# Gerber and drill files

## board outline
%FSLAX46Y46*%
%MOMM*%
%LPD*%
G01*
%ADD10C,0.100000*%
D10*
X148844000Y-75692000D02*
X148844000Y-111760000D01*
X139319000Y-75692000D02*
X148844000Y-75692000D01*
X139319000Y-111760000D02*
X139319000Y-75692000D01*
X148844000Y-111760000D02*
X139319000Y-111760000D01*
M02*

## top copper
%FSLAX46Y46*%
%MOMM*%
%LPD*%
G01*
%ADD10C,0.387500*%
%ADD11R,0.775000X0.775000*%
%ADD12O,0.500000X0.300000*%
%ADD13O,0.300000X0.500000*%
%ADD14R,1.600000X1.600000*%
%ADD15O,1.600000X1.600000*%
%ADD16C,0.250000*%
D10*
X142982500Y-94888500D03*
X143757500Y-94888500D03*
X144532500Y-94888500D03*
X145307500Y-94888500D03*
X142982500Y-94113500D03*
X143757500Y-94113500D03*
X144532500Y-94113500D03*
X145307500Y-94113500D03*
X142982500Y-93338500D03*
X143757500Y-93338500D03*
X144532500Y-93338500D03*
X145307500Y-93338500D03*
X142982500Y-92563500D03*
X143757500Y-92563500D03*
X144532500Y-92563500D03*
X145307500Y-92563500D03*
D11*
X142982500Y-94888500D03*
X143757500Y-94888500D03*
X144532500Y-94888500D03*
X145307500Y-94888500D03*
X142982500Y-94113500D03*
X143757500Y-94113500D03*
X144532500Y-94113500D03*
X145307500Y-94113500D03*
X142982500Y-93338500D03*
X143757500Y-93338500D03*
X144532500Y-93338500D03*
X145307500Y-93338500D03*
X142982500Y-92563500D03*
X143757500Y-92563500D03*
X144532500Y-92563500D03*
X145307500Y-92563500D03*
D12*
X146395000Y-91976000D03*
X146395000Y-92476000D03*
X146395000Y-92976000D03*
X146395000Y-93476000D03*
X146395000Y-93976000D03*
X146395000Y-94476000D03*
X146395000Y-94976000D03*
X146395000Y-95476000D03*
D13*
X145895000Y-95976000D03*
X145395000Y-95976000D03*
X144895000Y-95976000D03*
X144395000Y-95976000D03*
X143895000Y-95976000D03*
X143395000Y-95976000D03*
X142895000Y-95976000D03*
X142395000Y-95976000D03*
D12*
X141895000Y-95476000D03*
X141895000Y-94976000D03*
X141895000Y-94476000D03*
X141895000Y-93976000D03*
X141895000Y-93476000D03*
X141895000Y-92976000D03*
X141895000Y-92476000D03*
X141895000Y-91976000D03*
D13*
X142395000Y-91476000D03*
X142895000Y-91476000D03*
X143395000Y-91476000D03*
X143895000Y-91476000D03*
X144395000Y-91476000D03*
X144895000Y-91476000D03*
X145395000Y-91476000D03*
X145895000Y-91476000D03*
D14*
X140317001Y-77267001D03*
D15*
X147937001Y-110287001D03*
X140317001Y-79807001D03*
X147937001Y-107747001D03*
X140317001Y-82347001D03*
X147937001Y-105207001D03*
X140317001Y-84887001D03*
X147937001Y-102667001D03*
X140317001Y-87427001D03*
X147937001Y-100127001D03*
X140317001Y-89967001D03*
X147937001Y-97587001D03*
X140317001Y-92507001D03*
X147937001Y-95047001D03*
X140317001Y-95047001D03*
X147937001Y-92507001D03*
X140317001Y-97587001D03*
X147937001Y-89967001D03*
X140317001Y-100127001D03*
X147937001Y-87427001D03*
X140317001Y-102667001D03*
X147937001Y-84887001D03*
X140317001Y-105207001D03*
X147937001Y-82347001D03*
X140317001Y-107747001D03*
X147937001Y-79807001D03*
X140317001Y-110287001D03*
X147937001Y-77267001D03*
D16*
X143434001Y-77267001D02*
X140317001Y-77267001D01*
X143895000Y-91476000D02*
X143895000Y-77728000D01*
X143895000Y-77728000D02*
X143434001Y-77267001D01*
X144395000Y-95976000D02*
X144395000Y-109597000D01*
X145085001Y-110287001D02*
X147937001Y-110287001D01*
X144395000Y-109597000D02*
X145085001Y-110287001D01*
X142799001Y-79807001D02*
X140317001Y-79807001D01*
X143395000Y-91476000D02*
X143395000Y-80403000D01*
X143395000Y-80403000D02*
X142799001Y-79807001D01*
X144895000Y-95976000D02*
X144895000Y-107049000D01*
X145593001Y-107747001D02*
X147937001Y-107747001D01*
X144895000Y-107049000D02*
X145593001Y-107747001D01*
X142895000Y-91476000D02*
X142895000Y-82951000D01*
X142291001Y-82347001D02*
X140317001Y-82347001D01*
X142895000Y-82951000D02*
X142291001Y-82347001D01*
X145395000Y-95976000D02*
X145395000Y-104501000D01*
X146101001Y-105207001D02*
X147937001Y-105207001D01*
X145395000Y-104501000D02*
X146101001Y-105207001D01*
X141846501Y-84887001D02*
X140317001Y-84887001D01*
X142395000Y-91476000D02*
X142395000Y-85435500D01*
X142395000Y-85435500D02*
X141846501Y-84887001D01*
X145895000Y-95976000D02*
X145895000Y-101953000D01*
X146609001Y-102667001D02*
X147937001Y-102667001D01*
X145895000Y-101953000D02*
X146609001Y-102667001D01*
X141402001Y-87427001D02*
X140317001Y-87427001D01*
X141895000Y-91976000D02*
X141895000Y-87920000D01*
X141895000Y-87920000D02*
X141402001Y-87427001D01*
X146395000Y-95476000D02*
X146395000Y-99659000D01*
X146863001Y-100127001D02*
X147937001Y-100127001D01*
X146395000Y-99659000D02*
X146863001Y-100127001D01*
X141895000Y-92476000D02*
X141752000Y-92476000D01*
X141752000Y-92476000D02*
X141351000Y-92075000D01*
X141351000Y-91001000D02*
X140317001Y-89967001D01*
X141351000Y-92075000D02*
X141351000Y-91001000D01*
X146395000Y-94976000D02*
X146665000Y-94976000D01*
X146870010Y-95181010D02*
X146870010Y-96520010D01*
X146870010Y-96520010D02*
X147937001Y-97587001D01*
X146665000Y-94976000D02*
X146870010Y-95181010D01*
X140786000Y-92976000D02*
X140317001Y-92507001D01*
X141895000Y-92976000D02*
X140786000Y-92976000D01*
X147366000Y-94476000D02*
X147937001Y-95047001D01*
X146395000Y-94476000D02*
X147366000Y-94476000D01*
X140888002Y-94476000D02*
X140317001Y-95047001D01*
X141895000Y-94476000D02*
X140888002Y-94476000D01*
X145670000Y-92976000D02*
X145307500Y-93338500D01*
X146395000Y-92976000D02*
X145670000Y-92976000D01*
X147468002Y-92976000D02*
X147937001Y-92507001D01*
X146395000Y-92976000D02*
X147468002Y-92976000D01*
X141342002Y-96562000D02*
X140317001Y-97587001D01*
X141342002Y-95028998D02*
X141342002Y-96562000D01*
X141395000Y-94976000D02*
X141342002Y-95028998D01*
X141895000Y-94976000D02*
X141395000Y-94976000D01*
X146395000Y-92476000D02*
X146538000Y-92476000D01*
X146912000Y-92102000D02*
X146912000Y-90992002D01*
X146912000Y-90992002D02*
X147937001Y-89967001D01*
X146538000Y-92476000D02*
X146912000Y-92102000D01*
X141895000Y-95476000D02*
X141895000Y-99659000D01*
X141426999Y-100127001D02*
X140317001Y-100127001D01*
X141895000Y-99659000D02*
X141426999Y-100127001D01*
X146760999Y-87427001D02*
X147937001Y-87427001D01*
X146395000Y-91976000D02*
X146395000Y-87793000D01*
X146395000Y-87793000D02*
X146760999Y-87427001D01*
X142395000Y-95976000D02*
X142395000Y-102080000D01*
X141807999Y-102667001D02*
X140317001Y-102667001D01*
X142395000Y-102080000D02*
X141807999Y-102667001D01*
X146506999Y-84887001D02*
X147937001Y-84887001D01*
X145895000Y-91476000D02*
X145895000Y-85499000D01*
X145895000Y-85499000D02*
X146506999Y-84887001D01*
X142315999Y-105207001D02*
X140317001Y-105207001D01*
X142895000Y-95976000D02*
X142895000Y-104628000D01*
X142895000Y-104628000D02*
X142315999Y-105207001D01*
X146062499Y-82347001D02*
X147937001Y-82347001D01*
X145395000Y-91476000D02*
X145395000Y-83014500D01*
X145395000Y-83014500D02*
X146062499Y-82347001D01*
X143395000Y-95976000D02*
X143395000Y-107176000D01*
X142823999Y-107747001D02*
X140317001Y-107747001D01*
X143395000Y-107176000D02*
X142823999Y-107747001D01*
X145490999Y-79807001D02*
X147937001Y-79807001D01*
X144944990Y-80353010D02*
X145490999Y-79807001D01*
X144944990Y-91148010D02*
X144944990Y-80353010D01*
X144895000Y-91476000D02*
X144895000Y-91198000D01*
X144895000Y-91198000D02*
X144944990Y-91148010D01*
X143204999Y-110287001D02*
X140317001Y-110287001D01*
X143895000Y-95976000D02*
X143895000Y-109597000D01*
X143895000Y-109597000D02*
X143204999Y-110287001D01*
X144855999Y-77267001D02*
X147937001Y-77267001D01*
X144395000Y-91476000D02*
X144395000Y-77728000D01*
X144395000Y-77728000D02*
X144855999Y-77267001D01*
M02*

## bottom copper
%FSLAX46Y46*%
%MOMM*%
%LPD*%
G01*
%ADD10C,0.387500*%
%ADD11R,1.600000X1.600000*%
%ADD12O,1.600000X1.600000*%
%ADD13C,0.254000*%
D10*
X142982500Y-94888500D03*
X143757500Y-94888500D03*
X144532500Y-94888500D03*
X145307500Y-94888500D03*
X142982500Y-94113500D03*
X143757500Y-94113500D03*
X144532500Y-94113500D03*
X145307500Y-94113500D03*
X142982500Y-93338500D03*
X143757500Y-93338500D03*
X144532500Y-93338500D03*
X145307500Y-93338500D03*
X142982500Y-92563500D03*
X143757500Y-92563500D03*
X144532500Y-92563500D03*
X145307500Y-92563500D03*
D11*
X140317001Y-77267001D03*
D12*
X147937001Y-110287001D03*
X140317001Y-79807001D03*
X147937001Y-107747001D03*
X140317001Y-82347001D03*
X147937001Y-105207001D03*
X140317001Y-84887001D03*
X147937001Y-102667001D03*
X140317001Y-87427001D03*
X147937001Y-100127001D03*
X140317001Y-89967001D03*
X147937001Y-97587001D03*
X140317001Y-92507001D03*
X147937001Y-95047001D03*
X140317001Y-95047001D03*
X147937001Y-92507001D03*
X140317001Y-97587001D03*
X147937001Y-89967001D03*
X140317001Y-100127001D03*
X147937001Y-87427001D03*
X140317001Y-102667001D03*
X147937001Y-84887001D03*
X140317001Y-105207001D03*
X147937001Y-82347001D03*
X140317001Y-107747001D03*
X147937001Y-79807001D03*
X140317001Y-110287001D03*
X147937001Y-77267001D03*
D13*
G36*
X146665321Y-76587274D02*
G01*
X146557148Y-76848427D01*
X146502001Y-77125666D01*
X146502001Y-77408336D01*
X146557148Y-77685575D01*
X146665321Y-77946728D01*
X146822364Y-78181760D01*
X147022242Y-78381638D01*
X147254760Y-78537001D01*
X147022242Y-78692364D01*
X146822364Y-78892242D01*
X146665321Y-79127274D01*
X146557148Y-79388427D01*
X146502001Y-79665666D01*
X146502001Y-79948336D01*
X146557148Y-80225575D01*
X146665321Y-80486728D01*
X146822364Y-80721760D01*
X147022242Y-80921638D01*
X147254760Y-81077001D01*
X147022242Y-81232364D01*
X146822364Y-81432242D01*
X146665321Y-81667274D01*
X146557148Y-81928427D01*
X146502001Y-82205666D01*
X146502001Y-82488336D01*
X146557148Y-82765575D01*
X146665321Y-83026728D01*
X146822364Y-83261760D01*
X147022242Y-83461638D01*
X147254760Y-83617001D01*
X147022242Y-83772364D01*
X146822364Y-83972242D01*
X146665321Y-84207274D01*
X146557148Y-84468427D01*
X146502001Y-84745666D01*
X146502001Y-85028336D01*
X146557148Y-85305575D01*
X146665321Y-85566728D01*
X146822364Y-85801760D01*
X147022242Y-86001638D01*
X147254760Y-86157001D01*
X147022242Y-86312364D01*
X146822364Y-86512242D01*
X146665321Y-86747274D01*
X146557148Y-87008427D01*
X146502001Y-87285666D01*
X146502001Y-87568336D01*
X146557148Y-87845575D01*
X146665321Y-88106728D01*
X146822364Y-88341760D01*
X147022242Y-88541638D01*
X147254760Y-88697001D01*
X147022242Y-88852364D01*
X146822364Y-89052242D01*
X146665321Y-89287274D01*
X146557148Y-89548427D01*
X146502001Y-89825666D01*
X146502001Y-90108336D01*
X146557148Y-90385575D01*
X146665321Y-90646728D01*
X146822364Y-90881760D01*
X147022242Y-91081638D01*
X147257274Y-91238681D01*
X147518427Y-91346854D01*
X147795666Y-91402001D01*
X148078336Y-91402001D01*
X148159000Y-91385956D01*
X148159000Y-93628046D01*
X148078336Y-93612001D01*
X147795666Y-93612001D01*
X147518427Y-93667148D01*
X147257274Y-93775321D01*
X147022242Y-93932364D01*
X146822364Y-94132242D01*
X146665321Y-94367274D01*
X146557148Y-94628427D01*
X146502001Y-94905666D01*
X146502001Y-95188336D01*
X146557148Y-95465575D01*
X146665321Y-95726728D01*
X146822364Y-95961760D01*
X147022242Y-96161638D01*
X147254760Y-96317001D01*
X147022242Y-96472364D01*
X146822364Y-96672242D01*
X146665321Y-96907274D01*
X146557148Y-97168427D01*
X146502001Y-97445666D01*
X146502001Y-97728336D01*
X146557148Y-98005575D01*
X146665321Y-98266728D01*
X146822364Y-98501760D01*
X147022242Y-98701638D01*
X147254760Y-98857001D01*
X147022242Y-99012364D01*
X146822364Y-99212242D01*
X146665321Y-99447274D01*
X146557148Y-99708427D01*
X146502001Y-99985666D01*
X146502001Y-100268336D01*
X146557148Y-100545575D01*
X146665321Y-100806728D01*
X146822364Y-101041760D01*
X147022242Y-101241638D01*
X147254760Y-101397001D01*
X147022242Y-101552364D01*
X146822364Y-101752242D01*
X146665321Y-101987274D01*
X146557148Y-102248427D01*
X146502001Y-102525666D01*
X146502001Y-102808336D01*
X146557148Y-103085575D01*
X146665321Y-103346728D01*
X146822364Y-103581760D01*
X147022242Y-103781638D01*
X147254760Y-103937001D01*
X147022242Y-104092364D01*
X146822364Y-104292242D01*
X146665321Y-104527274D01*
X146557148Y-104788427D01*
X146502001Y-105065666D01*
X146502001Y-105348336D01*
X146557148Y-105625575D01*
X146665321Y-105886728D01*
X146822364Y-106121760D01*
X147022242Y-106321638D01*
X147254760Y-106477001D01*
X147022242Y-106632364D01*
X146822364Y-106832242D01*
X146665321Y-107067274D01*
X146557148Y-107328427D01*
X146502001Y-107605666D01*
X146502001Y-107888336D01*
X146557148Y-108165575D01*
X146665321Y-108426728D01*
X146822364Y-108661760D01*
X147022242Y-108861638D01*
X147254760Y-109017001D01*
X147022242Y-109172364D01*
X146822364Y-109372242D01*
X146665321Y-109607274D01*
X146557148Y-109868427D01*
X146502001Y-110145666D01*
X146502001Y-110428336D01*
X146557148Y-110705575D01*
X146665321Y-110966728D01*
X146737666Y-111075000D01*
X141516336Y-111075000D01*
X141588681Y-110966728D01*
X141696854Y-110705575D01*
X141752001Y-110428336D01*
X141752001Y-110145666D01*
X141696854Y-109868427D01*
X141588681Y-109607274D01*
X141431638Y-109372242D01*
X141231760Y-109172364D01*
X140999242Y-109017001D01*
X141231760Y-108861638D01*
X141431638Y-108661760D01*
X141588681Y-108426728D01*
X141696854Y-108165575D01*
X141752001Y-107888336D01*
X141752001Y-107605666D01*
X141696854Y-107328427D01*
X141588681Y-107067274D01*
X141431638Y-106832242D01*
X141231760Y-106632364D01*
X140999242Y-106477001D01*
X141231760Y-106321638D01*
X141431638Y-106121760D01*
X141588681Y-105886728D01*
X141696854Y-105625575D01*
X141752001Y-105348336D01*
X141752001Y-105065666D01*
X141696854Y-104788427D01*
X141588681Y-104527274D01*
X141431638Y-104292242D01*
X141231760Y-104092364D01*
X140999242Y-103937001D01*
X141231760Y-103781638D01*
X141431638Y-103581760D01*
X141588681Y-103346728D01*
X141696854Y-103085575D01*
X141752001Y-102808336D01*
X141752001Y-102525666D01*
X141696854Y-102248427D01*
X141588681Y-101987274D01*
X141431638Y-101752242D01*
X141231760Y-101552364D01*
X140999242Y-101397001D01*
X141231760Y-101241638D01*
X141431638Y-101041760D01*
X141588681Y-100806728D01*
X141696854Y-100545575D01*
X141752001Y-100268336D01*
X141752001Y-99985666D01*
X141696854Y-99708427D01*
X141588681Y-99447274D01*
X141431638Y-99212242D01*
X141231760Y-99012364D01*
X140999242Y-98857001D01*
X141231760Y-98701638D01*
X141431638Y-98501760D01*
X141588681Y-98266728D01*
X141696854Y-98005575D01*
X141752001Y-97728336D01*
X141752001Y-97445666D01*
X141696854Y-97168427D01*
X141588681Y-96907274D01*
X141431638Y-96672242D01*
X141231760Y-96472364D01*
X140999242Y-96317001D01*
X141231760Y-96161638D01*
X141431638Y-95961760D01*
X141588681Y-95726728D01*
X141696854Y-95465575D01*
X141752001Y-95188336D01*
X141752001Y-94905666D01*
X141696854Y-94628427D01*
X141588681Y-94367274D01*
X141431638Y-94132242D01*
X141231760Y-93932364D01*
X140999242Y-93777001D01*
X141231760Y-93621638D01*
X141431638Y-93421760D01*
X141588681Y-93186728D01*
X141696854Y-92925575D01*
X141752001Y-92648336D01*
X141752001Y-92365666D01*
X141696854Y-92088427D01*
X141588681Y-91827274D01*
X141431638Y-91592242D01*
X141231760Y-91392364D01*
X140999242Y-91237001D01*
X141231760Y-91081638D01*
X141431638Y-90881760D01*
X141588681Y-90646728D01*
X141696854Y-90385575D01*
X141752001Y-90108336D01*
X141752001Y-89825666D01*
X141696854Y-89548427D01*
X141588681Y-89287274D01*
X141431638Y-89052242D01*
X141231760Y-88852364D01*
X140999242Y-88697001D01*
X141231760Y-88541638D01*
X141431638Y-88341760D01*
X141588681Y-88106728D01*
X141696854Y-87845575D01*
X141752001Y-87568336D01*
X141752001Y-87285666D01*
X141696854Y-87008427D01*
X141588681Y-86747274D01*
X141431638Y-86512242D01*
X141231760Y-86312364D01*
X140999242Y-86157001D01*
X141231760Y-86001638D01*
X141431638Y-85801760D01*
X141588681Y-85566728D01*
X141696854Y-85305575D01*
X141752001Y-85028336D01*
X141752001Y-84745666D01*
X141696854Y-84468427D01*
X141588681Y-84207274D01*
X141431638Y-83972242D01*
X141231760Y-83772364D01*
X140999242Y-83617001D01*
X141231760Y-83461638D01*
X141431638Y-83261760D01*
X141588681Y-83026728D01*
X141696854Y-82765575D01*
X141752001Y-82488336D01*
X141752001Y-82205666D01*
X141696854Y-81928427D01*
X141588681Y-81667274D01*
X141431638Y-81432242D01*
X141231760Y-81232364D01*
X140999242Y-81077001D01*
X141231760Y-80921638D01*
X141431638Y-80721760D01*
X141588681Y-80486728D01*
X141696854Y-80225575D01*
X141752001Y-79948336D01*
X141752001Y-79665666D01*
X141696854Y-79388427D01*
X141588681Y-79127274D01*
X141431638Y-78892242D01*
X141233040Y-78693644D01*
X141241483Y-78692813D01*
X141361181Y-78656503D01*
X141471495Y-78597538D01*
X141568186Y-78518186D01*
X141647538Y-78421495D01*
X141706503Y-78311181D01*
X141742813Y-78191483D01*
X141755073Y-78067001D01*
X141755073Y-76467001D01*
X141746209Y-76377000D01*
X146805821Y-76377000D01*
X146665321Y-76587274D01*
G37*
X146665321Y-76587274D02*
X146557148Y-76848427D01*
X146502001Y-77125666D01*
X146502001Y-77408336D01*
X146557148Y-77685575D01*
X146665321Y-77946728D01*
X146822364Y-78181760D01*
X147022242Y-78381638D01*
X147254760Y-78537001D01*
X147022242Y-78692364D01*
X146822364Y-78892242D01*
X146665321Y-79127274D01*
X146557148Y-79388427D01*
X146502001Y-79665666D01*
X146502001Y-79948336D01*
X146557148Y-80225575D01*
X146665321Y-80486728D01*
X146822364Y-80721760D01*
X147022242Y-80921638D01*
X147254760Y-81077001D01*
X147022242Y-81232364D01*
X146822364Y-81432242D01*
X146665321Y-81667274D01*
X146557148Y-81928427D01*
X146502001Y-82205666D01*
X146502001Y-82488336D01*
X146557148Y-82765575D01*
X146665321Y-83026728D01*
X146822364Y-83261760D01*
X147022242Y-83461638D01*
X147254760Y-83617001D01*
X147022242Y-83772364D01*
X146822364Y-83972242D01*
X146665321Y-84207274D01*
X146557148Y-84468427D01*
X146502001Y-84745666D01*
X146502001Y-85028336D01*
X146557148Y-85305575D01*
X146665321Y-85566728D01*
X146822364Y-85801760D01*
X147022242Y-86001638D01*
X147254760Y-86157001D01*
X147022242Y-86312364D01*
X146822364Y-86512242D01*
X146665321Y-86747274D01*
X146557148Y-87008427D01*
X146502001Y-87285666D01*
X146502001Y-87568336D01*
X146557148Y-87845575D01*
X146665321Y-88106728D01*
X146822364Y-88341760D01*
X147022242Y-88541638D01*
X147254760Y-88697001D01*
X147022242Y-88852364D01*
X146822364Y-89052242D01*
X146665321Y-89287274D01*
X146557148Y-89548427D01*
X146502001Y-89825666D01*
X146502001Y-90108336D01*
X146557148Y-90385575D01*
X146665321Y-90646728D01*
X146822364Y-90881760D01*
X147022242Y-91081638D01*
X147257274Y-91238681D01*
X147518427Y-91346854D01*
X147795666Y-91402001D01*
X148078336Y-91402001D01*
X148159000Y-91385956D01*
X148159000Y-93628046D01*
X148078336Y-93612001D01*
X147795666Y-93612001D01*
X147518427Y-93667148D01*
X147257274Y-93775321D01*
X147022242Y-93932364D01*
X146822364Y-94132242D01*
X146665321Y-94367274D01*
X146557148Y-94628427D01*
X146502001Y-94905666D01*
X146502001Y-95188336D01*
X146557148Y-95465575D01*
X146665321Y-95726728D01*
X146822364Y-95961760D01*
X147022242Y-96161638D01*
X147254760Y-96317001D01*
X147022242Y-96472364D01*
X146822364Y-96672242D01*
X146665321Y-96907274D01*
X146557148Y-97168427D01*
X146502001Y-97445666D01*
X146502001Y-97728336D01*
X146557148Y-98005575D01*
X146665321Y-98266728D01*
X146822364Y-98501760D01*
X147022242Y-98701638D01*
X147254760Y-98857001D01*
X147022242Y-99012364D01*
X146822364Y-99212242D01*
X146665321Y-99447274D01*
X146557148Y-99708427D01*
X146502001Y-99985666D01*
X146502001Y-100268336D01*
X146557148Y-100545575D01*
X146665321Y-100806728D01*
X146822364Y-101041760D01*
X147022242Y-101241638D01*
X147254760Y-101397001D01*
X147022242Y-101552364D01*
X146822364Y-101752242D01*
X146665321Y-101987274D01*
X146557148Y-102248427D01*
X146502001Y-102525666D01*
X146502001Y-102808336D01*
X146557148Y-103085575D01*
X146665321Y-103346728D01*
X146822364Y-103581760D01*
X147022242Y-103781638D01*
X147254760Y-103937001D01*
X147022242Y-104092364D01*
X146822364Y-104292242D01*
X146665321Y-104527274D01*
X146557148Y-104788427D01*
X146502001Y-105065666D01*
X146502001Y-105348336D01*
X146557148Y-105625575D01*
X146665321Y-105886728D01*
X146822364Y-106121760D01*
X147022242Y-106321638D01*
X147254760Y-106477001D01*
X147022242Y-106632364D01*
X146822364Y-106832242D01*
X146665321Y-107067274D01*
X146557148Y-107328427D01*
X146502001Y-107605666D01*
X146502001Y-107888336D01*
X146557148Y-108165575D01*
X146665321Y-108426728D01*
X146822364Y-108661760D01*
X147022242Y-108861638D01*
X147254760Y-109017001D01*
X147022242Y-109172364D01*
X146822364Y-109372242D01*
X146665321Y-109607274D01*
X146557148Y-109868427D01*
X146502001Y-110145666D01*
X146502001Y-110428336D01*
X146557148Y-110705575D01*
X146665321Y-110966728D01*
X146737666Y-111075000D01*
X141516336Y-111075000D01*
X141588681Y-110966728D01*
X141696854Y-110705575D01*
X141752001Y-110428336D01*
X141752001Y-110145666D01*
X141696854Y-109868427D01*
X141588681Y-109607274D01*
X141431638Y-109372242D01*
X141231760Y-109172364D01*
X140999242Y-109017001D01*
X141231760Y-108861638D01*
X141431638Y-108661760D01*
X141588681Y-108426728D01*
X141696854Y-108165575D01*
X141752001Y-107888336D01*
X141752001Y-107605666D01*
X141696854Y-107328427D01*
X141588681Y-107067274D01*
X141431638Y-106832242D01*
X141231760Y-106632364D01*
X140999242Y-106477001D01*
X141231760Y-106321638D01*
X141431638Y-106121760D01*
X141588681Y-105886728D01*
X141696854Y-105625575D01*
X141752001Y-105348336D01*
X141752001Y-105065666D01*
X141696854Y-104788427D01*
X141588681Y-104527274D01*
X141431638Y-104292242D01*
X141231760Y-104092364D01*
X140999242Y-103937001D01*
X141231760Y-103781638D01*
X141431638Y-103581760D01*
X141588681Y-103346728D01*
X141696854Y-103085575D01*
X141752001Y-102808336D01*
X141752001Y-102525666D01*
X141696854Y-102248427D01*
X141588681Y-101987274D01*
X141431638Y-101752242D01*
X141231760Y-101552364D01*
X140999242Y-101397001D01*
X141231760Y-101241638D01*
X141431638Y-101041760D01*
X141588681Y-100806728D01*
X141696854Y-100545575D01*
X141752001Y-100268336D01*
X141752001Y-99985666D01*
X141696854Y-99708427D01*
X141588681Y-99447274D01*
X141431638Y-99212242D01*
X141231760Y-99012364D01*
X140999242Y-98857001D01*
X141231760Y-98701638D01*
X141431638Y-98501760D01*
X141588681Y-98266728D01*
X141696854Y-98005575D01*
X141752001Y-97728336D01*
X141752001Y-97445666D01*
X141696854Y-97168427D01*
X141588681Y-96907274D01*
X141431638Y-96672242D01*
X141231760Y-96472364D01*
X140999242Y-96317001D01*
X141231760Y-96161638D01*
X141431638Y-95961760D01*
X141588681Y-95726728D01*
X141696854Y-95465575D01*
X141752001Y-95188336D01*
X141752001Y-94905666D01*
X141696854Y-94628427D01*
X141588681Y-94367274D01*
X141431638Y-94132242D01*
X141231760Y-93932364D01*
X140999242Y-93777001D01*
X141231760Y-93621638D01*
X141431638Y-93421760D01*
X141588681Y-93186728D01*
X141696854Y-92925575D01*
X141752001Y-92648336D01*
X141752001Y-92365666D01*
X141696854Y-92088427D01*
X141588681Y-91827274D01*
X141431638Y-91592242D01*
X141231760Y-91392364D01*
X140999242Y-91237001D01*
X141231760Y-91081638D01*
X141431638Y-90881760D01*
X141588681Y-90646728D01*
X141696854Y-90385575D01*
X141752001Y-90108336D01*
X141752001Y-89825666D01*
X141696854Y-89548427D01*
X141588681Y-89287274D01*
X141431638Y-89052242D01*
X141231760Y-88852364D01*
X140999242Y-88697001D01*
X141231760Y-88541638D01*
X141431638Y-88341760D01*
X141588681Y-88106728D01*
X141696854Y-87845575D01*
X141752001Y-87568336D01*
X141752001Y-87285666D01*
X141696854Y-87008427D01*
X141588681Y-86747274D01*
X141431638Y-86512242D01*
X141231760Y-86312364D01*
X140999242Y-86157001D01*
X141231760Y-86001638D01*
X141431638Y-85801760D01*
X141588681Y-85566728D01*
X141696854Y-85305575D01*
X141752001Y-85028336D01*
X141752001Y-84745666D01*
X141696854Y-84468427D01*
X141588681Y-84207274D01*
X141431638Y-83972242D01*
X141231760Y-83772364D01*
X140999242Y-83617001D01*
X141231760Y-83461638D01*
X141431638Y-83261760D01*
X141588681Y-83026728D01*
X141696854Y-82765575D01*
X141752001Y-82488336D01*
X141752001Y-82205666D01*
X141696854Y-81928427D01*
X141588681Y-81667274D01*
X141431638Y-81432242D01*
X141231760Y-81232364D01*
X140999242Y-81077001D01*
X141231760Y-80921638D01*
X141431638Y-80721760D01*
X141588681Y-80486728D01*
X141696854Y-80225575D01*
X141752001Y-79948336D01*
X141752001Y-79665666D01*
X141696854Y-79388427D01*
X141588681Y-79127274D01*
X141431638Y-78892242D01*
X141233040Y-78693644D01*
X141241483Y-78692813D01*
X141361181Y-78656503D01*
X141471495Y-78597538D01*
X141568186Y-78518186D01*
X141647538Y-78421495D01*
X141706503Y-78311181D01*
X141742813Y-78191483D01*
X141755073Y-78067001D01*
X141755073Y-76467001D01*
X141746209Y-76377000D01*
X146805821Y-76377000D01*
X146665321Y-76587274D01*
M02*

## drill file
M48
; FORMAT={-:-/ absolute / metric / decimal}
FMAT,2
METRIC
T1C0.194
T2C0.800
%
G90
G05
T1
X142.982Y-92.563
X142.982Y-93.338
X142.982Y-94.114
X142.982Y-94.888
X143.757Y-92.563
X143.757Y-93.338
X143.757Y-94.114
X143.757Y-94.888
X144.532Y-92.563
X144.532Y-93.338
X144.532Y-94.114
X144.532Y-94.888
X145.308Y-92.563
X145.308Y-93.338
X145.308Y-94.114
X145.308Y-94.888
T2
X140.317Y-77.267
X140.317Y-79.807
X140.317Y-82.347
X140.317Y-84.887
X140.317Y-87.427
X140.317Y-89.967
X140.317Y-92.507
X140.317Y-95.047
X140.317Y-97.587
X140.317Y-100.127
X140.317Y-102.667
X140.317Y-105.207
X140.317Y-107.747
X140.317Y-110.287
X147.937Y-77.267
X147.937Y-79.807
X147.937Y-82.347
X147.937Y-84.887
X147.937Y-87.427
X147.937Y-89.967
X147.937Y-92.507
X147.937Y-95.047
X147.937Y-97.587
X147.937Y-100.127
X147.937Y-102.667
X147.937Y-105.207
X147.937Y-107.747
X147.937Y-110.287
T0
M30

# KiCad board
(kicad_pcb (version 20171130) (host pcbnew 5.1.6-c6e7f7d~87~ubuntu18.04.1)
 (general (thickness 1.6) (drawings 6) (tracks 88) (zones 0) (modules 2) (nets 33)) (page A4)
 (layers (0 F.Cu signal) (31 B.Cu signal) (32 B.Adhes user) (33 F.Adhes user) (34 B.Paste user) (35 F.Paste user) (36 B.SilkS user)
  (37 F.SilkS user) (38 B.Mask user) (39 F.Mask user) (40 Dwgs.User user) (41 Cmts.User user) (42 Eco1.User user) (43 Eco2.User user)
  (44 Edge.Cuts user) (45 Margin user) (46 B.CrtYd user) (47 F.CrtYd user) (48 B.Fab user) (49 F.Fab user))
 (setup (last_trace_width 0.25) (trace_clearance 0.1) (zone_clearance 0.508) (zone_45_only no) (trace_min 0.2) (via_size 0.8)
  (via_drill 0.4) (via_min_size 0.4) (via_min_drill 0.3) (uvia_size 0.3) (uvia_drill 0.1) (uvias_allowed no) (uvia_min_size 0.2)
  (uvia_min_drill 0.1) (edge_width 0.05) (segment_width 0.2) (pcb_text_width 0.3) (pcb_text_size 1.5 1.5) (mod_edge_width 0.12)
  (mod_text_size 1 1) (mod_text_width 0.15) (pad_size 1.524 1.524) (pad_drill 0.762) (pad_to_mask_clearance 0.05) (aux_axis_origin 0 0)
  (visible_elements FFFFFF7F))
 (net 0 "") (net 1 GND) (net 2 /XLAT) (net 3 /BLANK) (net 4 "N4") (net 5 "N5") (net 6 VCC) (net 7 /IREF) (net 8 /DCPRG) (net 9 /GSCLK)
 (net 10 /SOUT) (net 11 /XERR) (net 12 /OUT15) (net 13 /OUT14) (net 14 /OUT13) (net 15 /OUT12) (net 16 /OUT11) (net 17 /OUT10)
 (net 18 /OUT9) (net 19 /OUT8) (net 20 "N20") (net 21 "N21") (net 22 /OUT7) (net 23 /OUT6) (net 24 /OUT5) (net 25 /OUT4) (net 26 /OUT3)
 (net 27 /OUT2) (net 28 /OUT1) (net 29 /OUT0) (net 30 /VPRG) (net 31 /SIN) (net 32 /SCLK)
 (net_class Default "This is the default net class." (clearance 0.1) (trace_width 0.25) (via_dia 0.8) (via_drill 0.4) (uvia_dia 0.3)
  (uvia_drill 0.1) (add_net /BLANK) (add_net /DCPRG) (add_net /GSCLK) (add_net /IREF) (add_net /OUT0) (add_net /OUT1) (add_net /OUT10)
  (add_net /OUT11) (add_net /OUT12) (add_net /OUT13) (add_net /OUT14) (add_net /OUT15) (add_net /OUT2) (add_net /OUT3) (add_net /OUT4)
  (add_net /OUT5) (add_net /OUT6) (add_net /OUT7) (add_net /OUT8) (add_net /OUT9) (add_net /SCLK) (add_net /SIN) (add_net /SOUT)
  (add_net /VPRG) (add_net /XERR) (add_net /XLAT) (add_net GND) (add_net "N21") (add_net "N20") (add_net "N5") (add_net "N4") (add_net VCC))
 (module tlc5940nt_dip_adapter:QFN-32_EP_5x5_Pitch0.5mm (layer F.Cu) (at 144.145 93.726 270)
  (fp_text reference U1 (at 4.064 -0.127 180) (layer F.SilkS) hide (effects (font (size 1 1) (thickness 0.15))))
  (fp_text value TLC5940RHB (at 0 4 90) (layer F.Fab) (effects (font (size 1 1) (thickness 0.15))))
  (pad 33 thru_hole circle (at 1.1625 1.1625 270) (size 0.3875 0.3875) (drill 0.19375) (layers *.Cu *.Mask) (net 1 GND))
  (pad 33 thru_hole circle (at 1.1625 0.3875 270) (size 0.3875 0.3875) (drill 0.19375) (layers *.Cu *.Mask) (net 1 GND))
  (pad 33 thru_hole circle (at 1.1625 -0.3875 270) (size 0.3875 0.3875) (drill 0.19375) (layers *.Cu *.Mask) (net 1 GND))
  (pad 33 thru_hole circle (at 1.1625 -1.1625 270) (size 0.3875 0.3875) (drill 0.19375) (layers *.Cu *.Mask) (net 1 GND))
  (pad 33 thru_hole circle (at 0.3875 1.1625 270) (size 0.3875 0.3875) (drill 0.19375) (layers *.Cu *.Mask) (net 1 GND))
  (pad 33 thru_hole circle (at 0.3875 0.3875 270) (size 0.3875 0.3875) (drill 0.19375) (layers *.Cu *.Mask) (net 1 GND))
  (pad 33 thru_hole circle (at 0.3875 -0.3875 270) (size 0.3875 0.3875) (drill 0.19375) (layers *.Cu *.Mask) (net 1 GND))
  (pad 33 thru_hole circle (at 0.3875 -1.1625 270) (size 0.3875 0.3875) (drill 0.19375) (layers *.Cu *.Mask) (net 1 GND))
  (pad 33 thru_hole circle (at -0.3875 1.1625 270) (size 0.3875 0.3875) (drill 0.19375) (layers *.Cu *.Mask) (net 1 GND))
  (pad 33 thru_hole circle (at -0.3875 0.3875 270) (size 0.3875 0.3875) (drill 0.19375) (layers *.Cu *.Mask) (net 1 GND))
  (pad 33 thru_hole circle (at -0.3875 -0.3875 270) (size 0.3875 0.3875) (drill 0.19375) (layers *.Cu *.Mask) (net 1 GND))
  (pad 33 thru_hole circle (at -0.3875 -1.1625 270) (size 0.3875 0.3875) (drill 0.19375) (layers *.Cu *.Mask) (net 1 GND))
  (pad 33 thru_hole circle (at -1.1625 1.1625 270) (size 0.3875 0.3875) (drill 0.19375) (layers *.Cu *.Mask) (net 1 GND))
  (pad 33 thru_hole circle (at -1.1625 0.3875 270) (size 0.3875 0.3875) (drill 0.19375) (layers *.Cu *.Mask) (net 1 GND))
  (pad 33 thru_hole circle (at -1.1625 -0.3875 270) (size 0.3875 0.3875) (drill 0.19375) (layers *.Cu *.Mask) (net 1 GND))
  (pad 33 thru_hole circle (at -1.1625 -1.1625 270) (size 0.3875 0.3875) (drill 0.19375) (layers *.Cu *.Mask) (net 1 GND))
  (pad 33 smd rect (at 1.1625 1.1625 270) (size 0.775 0.775) (layers F.Cu F.Paste F.Mask) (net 1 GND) (solder_paste_margin -0.75))
  (pad 33 smd rect (at 1.1625 0.3875 270) (size 0.775 0.775) (layers F.Cu F.Paste F.Mask) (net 1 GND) (solder_paste_margin -0.75))
  (pad 33 smd rect (at 1.1625 -0.3875 270) (size 0.775 0.775) (layers F.Cu F.Paste F.Mask) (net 1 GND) (solder_paste_margin -0.75))
  (pad 33 smd rect (at 1.1625 -1.1625 270) (size 0.775 0.775) (layers F.Cu F.Paste F.Mask) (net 1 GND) (solder_paste_margin -0.75))
  (pad 33 smd rect (at 0.3875 1.1625 270) (size 0.775 0.775) (layers F.Cu F.Paste F.Mask) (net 1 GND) (solder_paste_margin -0.75))
  (pad 33 smd rect (at 0.3875 0.3875 270) (size 0.775 0.775) (layers F.Cu F.Paste F.Mask) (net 1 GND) (solder_paste_margin -0.75))
  (pad 33 smd rect (at 0.3875 -0.3875 270) (size 0.775 0.775) (layers F.Cu F.Paste F.Mask) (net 1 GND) (solder_paste_margin -0.75))
  (pad 33 smd rect (at 0.3875 -1.1625 270) (size 0.775 0.775) (layers F.Cu F.Paste F.Mask) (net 1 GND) (solder_paste_margin -0.75))
  (pad 33 smd rect (at -0.3875 1.1625 270) (size 0.775 0.775) (layers F.Cu F.Paste F.Mask) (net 1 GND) (solder_paste_margin -0.75))
  (pad 33 smd rect (at -0.3875 0.3875 270) (size 0.775 0.775) (layers F.Cu F.Paste F.Mask) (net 1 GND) (solder_paste_margin -0.75))
  (pad 33 smd rect (at -0.3875 -0.3875 270) (size 0.775 0.775) (layers F.Cu F.Paste F.Mask) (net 1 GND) (solder_paste_margin -0.75))
  (pad 33 smd rect (at -0.3875 -1.1625 270) (size 0.775 0.775) (layers F.Cu F.Paste F.Mask) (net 1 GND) (solder_paste_margin -0.75))
  (pad 33 smd rect (at -1.1625 1.1625 270) (size 0.775 0.775) (layers F.Cu F.Paste F.Mask) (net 1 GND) (solder_paste_margin -0.75))
  (pad 33 smd rect (at -1.1625 0.3875 270) (size 0.775 0.775) (layers F.Cu F.Paste F.Mask) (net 1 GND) (solder_paste_margin -0.75))
  (pad 33 smd rect (at -1.1625 -0.3875 270) (size 0.775 0.775) (layers F.Cu F.Paste F.Mask) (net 1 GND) (solder_paste_margin -0.75))
  (pad 33 smd rect (at -1.1625 -1.1625 270) (size 0.775 0.775) (layers F.Cu F.Paste F.Mask) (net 1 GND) (solder_paste_margin -0.75))
  (pad 32 smd oval (at -1.75 -2.25 270) (size 0.3 0.5) (layers F.Cu F.Paste F.Mask) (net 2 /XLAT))
  (pad 31 smd oval (at -1.25 -2.25 270) (size 0.3 0.5) (layers F.Cu F.Paste F.Mask) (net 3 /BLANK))
  (pad 30 smd oval (at -0.75 -2.25 270) (size 0.3 0.5) (layers F.Cu F.Paste F.Mask) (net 1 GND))
  (pad 29 smd oval (at -0.25 -2.25 270) (size 0.3 0.5) (layers F.Cu F.Paste F.Mask) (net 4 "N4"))
  (pad 28 smd oval (at 0.25 -2.25 270) (size 0.3 0.5) (layers F.Cu F.Paste F.Mask) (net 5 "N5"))
  (pad 27 smd oval (at 0.75 -2.25 270) (size 0.3 0.5) (layers F.Cu F.Paste F.Mask) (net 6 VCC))
  (pad 26 smd oval (at 1.25 -2.25 270) (size 0.3 0.5) (layers F.Cu F.Paste F.Mask) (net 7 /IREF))
  (pad 25 smd oval (at 1.75 -2.25 270) (size 0.3 0.5) (layers F.Cu F.Paste F.Mask) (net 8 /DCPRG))
  (pad 24 smd oval (at 2.25 -1.75) (size 0.3 0.5) (layers F.Cu F.Paste F.Mask) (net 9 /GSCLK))
  (pad 23 smd oval (at 2.25 -1.25) (size 0.3 0.5) (layers F.Cu F.Paste F.Mask) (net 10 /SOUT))
  (pad 22 smd oval (at 2.25 -0.75) (size 0.3 0.5) (layers F.Cu F.Paste F.Mask) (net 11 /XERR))
  (pad 21 smd oval (at 2.25 -0.25) (size 0.3 0.5) (layers F.Cu F.Paste F.Mask) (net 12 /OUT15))
  (pad 20 smd oval (at 2.25 0.25) (size 0.3 0.5) (layers F.Cu F.Paste F.Mask) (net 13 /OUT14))
  (pad 19 smd oval (at 2.25 0.75) (size 0.3 0.5) (layers F.Cu F.Paste F.Mask) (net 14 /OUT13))
  (pad 18 smd oval (at 2.25 1.25) (size 0.3 0.5) (layers F.Cu F.Paste F.Mask) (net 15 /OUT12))
  (pad 17 smd oval (at 2.25 1.75) (size 0.3 0.5) (layers F.Cu F.Paste F.Mask) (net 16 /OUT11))
  (pad 16 smd oval (at 1.75 2.25 270) (size 0.3 0.5) (layers F.Cu F.Paste F.Mask) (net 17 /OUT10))
  (pad 15 smd oval (at 1.25 2.25 270) (size 0.3 0.5) (layers F.Cu F.Paste F.Mask) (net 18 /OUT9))
  (pad 14 smd oval (at 0.75 2.25 270) (size 0.3 0.5) (layers F.Cu F.Paste F.Mask) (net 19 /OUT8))
  (pad 13 smd oval (at 0.25 2.25 270) (size 0.3 0.5) (layers F.Cu F.Paste F.Mask) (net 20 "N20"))
  (pad 12 smd oval (at -0.25 2.25 270) (size 0.3 0.5) (layers F.Cu F.Paste F.Mask) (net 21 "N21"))
  (pad 11 smd oval (at -0.75 2.25 270) (size 0.3 0.5) (layers F.Cu F.Paste F.Mask) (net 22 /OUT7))
  (pad 10 smd oval (at -1.25 2.25 270) (size 0.3 0.5) (layers F.Cu F.Paste F.Mask) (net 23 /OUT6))
  (pad 9 smd oval (at -1.75 2.25 270) (size 0.3 0.5) (layers F.Cu F.Paste F.Mask) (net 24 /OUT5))
  (pad 8 smd oval (at -2.25 1.75) (size 0.3 0.5) (layers F.Cu F.Paste F.Mask) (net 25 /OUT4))
  (pad 7 smd oval (at -2.25 1.25) (size 0.3 0.5) (layers F.Cu F.Paste F.Mask) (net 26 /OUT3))
  (pad 6 smd oval (at -2.25 0.75) (size 0.3 0.5) (layers F.Cu F.Paste F.Mask) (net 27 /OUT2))
  (pad 5 smd oval (at -2.25 0.25) (size 0.3 0.5) (layers F.Cu F.Paste F.Mask) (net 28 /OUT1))
  (pad 4 smd oval (at -2.25 -0.25) (size 0.3 0.5) (layers F.Cu F.Paste F.Mask) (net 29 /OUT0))
  (pad 3 smd oval (at -2.25 -0.75) (size 0.3 0.5) (layers F.Cu F.Paste F.Mask) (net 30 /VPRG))
  (pad 2 smd oval (at -2.25 -1.25) (size 0.3 0.5) (layers F.Cu F.Paste F.Mask) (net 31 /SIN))
  (pad 1 smd oval (at -2.25 -1.75) (size 0.3 0.5) (layers F.Cu F.Paste F.Mask) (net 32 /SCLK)))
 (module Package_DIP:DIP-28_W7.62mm (layer F.Cu) (at 140.317001 77.267001)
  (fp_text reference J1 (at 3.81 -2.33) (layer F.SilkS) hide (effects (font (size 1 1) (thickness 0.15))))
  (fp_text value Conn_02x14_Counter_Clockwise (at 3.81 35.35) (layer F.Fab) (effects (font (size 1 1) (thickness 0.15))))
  (pad 1 thru_hole rect (at 0 0) (size 1.6 1.6) (drill 0.8) (layers *.Cu *.Mask) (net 28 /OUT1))
  (pad 15 thru_hole oval (at 7.62 33.02) (size 1.6 1.6) (drill 0.8) (layers *.Cu *.Mask) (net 12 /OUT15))
  (pad 2 thru_hole oval (at 0 2.54) (size 1.6 1.6) (drill 0.8) (layers *.Cu *.Mask) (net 27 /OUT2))
  (pad 16 thru_hole oval (at 7.62 30.48) (size 1.6 1.6) (drill 0.8) (layers *.Cu *.Mask) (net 11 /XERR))
  (pad 3 thru_hole oval (at 0 5.08) (size 1.6 1.6) (drill 0.8) (layers *.Cu *.Mask) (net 26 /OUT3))
  (pad 17 thru_hole oval (at 7.62 27.94) (size 1.6 1.6) (drill 0.8) (layers *.Cu *.Mask) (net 10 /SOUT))
  (pad 4 thru_hole oval (at 0 7.62) (size 1.6 1.6) (drill 0.8) (layers *.Cu *.Mask) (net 25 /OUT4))
  (pad 18 thru_hole oval (at 7.62 25.4) (size 1.6 1.6) (drill 0.8) (layers *.Cu *.Mask) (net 9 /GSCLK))
  (pad 5 thru_hole oval (at 0 10.16) (size 1.6 1.6) (drill 0.8) (layers *.Cu *.Mask) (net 24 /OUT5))
  (pad 19 thru_hole oval (at 7.62 22.86) (size 1.6 1.6) (drill 0.8) (layers *.Cu *.Mask) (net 8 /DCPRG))
  (pad 6 thru_hole oval (at 0 12.7) (size 1.6 1.6) (drill 0.8) (layers *.Cu *.Mask) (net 23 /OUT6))
  (pad 20 thru_hole oval (at 7.62 20.32) (size 1.6 1.6) (drill 0.8) (layers *.Cu *.Mask) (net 7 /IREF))
  (pad 7 thru_hole oval (at 0 15.24) (size 1.6 1.6) (drill 0.8) (layers *.Cu *.Mask) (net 22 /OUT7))
  (pad 21 thru_hole oval (at 7.62 17.78) (size 1.6 1.6) (drill 0.8) (layers *.Cu *.Mask) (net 6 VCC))
  (pad 8 thru_hole oval (at 0 17.78) (size 1.6 1.6) (drill 0.8) (layers *.Cu *.Mask) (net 19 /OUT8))
  (pad 22 thru_hole oval (at 7.62 15.24) (size 1.6 1.6) (drill 0.8) (layers *.Cu *.Mask) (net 1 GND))
  (pad 9 thru_hole oval (at 0 20.32) (size 1.6 1.6) (drill 0.8) (layers *.Cu *.Mask) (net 18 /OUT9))
  (pad 23 thru_hole oval (at 7.62 12.7) (size 1.6 1.6) (drill 0.8) (layers *.Cu *.Mask) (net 3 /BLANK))
  (pad 10 thru_hole oval (at 0 22.86) (size 1.6 1.6) (drill 0.8) (layers *.Cu *.Mask) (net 17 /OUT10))
  (pad 24 thru_hole oval (at 7.62 10.16) (size 1.6 1.6) (drill 0.8) (layers *.Cu *.Mask) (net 2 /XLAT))
  (pad 11 thru_hole oval (at 0 25.4) (size 1.6 1.6) (drill 0.8) (layers *.Cu *.Mask) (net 16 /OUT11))
  (pad 25 thru_hole oval (at 7.62 7.62) (size 1.6 1.6) (drill 0.8) (layers *.Cu *.Mask) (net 32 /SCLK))
  (pad 12 thru_hole oval (at 0 27.94) (size 1.6 1.6) (drill 0.8) (layers *.Cu *.Mask) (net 15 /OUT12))
  (pad 26 thru_hole oval (at 7.62 5.08) (size 1.6 1.6) (drill 0.8) (layers *.Cu *.Mask) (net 31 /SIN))
  (pad 13 thru_hole oval (at 0 30.48) (size 1.6 1.6) (drill 0.8) (layers *.Cu *.Mask) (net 14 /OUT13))
  (pad 27 thru_hole oval (at 7.62 2.54) (size 1.6 1.6) (drill 0.8) (layers *.Cu *.Mask) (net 30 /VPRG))
  (pad 14 thru_hole oval (at 0 33.02) (size 1.6 1.6) (drill 0.8) (layers *.Cu *.Mask) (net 13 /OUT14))
  (pad 28 thru_hole oval (at 7.62 0) (size 1.6 1.6) (drill 0.8) (layers *.Cu *.Mask) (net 29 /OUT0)))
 (gr_line (start 148.844 75.692) (end 148.844 111.76) (layer Edge.Cuts) (width 0.1))
 (gr_line (start 139.319 75.692) (end 148.844 75.692) (layer Edge.Cuts) (width 0.1))
 (gr_line (start 139.319 111.76) (end 139.319 75.692) (layer Edge.Cuts) (width 0.1))
 (gr_line (start 148.844 111.76) (end 139.319 111.76) (layer Edge.Cuts) (width 0.1))
 (segment (start 143.434001 77.267001) (end 140.317001 77.267001) (width 0.25) (layer F.Cu) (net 28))
 (segment (start 143.895 91.476) (end 143.895 77.728) (width 0.25) (layer F.Cu) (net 28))
 (segment (start 143.895 77.728) (end 143.434001 77.267001) (width 0.25) (layer F.Cu) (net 28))
 (segment (start 144.395 95.976) (end 144.395 109.597) (width 0.25) (layer F.Cu) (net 12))
 (segment (start 145.085001 110.287001) (end 147.937001 110.287001) (width 0.25) (layer F.Cu) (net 12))
 (segment (start 144.395 109.597) (end 145.085001 110.287001) (width 0.25) (layer F.Cu) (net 12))
 (segment (start 142.799001 79.807001) (end 140.317001 79.807001) (width 0.25) (layer F.Cu) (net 27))
 (segment (start 143.395 91.476) (end 143.395 80.403) (width 0.25) (layer F.Cu) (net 27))
 (segment (start 143.395 80.403) (end 142.799001 79.807001) (width 0.25) (layer F.Cu) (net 27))
 (segment (start 144.895 95.976) (end 144.895 107.049) (width 0.25) (layer F.Cu) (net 11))
 (segment (start 145.593001 107.747001) (end 147.937001 107.747001) (width 0.25) (layer F.Cu) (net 11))
 (segment (start 144.895 107.049) (end 145.593001 107.747001) (width 0.25) (layer F.Cu) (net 11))
 (segment (start 142.895 91.476) (end 142.895 82.951) (width 0.25) (layer F.Cu) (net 26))
 (segment (start 142.291001 82.347001) (end 140.317001 82.347001) (width 0.25) (layer F.Cu) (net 26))
 (segment (start 142.895 82.951) (end 142.291001 82.347001) (width 0.25) (layer F.Cu) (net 26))
 (segment (start 145.395 95.976) (end 145.395 104.501) (width 0.25) (layer F.Cu) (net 10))
 (segment (start 146.101001 105.207001) (end 147.937001 105.207001) (width 0.25) (layer F.Cu) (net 10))
 (segment (start 145.395 104.501) (end 146.101001 105.207001) (width 0.25) (layer F.Cu) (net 10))
 (segment (start 141.846501 84.887001) (end 140.317001 84.887001) (width 0.25) (layer F.Cu) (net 25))
 (segment (start 142.395 91.476) (end 142.395 85.4355) (width 0.25) (layer F.Cu) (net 25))
 (segment (start 142.395 85.4355) (end 141.846501 84.887001) (width 0.25) (layer F.Cu) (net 25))
 (segment (start 145.895 95.976) (end 145.895 101.953) (width 0.25) (layer F.Cu) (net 9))
 (segment (start 146.609001 102.667001) (end 147.937001 102.667001) (width 0.25) (layer F.Cu) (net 9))
 (segment (start 145.895 101.953) (end 146.609001 102.667001) (width 0.25) (layer F.Cu) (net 9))
 (segment (start 141.402001 87.427001) (end 140.317001 87.427001) (width 0.25) (layer F.Cu) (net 24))
 (segment (start 141.895 91.976) (end 141.895 87.92) (width 0.25) (layer F.Cu) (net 24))
 (segment (start 141.895 87.92) (end 141.402001 87.427001) (width 0.25) (layer F.Cu) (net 24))
 (segment (start 146.395 95.476) (end 146.395 99.659) (width 0.25) (layer F.Cu) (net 8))
 (segment (start 146.863001 100.127001) (end 147.937001 100.127001) (width 0.25) (layer F.Cu) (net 8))
 (segment (start 146.395 99.659) (end 146.863001 100.127001) (width 0.25) (layer F.Cu) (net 8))
 (segment (start 141.895 92.476) (end 141.752 92.476) (width 0.25) (layer F.Cu) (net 23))
 (segment (start 141.752 92.476) (end 141.351 92.075) (width 0.25) (layer F.Cu) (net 23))
 (segment (start 141.351 91.001) (end 140.317001 89.967001) (width 0.25) (layer F.Cu) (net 23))
 (segment (start 141.351 92.075) (end 141.351 91.001) (width 0.25) (layer F.Cu) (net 23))
 (segment (start 146.395 94.976) (end 146.665 94.976) (width 0.25) (layer F.Cu) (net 7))
 (segment (start 146.87001 95.18101) (end 146.87001 96.52001) (width 0.25) (layer F.Cu) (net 7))
 (segment (start 146.87001 96.52001) (end 147.937001 97.587001) (width 0.25) (layer F.Cu) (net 7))
 (segment (start 146.665 94.976) (end 146.87001 95.18101) (width 0.25) (layer F.Cu) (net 7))
 (segment (start 140.786 92.976) (end 140.317001 92.507001) (width 0.25) (layer F.Cu) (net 22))
 (segment (start 141.895 92.976) (end 140.786 92.976) (width 0.25) (layer F.Cu) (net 22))
 (segment (start 147.366 94.476) (end 147.937001 95.047001) (width 0.25) (layer F.Cu) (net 6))
 (segment (start 146.395 94.476) (end 147.366 94.476) (width 0.25) (layer F.Cu) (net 6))
 (segment (start 140.888002 94.476) (end 140.317001 95.047001) (width 0.25) (layer F.Cu) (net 19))
 (segment (start 141.895 94.476) (end 140.888002 94.476) (width 0.25) (layer F.Cu) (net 19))
 (segment (start 145.67 92.976) (end 145.3075 93.3385) (width 0.25) (layer F.Cu) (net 1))
 (segment (start 146.395 92.976) (end 145.67 92.976) (width 0.25) (layer F.Cu) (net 1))
 (segment (start 147.468002 92.976) (end 147.937001 92.507001) (width 0.25) (layer F.Cu) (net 1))
 (segment (start 146.395 92.976) (end 147.468002 92.976) (width 0.25) (layer F.Cu) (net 1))
 (segment (start 141.342002 96.562) (end 140.317001 97.587001) (width 0.25) (layer F.Cu) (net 18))
 (segment (start 141.342002 95.028998) (end 141.342002 96.562) (width 0.25) (layer F.Cu) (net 18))
 (segment (start 141.395 94.976) (end 141.342002 95.028998) (width 0.25) (layer F.Cu) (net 18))
 (segment (start 141.895 94.976) (end 141.395 94.976) (width 0.25) (layer F.Cu) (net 18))
 (segment (start 146.395 92.476) (end 146.538 92.476) (width 0.25) (layer F.Cu) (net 3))
 (segment (start 146.912 92.102) (end 146.912 90.992002) (width 0.25) (layer F.Cu) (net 3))
 (segment (start 146.912 90.992002) (end 147.937001 89.967001) (width 0.25) (layer F.Cu) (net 3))
 (segment (start 146.538 92.476) (end 146.912 92.102) (width 0.25) (layer F.Cu) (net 3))
 (segment (start 141.895 95.476) (end 141.895 99.659) (width 0.25) (layer F.Cu) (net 17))
 (segment (start 141.426999 100.127001) (end 140.317001 100.127001) (width 0.25) (layer F.Cu) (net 17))
 (segment (start 141.895 99.659) (end 141.426999 100.127001) (width 0.25) (layer F.Cu) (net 17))
 (segment (start 146.760999 87.427001) (end 147.937001 87.427001) (width 0.25) (layer F.Cu) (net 2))
 (segment (start 146.395 91.976) (end 146.395 87.793) (width 0.25) (layer F.Cu) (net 2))
 (segment (start 146.395 87.793) (end 146.760999 87.427001) (width 0.25) (layer F.Cu) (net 2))
 (segment (start 142.395 95.976) (end 142.395 102.08) (width 0.25) (layer F.Cu) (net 16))
 (segment (start 141.807999 102.667001) (end 140.317001 102.667001) (width 0.25) (layer F.Cu) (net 16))
 (segment (start 142.395 102.08) (end 141.807999 102.667001) (width 0.25) (layer F.Cu) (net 16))
 (segment (start 146.506999 84.887001) (end 147.937001 84.887001) (width 0.25) (layer F.Cu) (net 32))
 (segment (start 145.895 91.476) (end 145.895 85.499) (width 0.25) (layer F.Cu) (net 32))
 (segment (start 145.895 85.499) (end 146.506999 84.887001) (width 0.25) (layer F.Cu) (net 32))
 (segment (start 142.315999 105.207001) (end 140.317001 105.207001) (width 0.25) (layer F.Cu) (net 15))
 (segment (start 142.895 95.976) (end 142.895 104.628) (width 0.25) (layer F.Cu) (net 15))
 (segment (start 142.895 104.628) (end 142.315999 105.207001) (width 0.25) (layer F.Cu) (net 15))
 (segment (start 146.062499 82.347001) (end 147.937001 82.347001) (width 0.25) (layer F.Cu) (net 31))
 (segment (start 145.395 91.476) (end 145.395 83.0145) (width 0.25) (layer F.Cu) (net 31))
 (segment (start 145.395 83.0145) (end 146.062499 82.347001) (width 0.25) (layer F.Cu) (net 31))
 (segment (start 143.395 95.976) (end 143.395 107.176) (width 0.25) (layer F.Cu) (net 14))
 (segment (start 142.823999 107.747001) (end 140.317001 107.747001) (width 0.25) (layer F.Cu) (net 14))
 (segment (start 143.395 107.176) (end 142.823999 107.747001) (width 0.25) (layer F.Cu) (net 14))
 (segment (start 145.490999 79.807001) (end 147.937001 79.807001) (width 0.25) (layer F.Cu) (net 30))
 (segment (start 144.94499 80.35301) (end 145.490999 79.807001) (width 0.25) (layer F.Cu) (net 30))
 (segment (start 144.94499 91.14801) (end 144.94499 80.35301) (width 0.25) (layer F.Cu) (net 30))
 (segment (start 144.895 91.476) (end 144.895 91.198) (width 0.25) (layer F.Cu) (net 30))
 (segment (start 144.895 91.198) (end 144.94499 91.14801) (width 0.25) (layer F.Cu) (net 30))
 (segment (start 143.204999 110.287001) (end 140.317001 110.287001) (width 0.25) (layer F.Cu) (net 13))
 (segment (start 143.895 95.976) (end 143.895 109.597) (width 0.25) (layer F.Cu) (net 13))
 (segment (start 143.895 109.597) (end 143.204999 110.287001) (width 0.25) (layer F.Cu) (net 13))
 (segment (start 144.855999 77.267001) (end 147.937001 77.267001) (width 0.25) (layer F.Cu) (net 29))
 (segment (start 144.395 91.476) (end 144.395 77.728) (width 0.25) (layer F.Cu) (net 29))
 (segment (start 144.395 77.728) (end 144.855999 77.267001) (width 0.25) (layer F.Cu) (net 29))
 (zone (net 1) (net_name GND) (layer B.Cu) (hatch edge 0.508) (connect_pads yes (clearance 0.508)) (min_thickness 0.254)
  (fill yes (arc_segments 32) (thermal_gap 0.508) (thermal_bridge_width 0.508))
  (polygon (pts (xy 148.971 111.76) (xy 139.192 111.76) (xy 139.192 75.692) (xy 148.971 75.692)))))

